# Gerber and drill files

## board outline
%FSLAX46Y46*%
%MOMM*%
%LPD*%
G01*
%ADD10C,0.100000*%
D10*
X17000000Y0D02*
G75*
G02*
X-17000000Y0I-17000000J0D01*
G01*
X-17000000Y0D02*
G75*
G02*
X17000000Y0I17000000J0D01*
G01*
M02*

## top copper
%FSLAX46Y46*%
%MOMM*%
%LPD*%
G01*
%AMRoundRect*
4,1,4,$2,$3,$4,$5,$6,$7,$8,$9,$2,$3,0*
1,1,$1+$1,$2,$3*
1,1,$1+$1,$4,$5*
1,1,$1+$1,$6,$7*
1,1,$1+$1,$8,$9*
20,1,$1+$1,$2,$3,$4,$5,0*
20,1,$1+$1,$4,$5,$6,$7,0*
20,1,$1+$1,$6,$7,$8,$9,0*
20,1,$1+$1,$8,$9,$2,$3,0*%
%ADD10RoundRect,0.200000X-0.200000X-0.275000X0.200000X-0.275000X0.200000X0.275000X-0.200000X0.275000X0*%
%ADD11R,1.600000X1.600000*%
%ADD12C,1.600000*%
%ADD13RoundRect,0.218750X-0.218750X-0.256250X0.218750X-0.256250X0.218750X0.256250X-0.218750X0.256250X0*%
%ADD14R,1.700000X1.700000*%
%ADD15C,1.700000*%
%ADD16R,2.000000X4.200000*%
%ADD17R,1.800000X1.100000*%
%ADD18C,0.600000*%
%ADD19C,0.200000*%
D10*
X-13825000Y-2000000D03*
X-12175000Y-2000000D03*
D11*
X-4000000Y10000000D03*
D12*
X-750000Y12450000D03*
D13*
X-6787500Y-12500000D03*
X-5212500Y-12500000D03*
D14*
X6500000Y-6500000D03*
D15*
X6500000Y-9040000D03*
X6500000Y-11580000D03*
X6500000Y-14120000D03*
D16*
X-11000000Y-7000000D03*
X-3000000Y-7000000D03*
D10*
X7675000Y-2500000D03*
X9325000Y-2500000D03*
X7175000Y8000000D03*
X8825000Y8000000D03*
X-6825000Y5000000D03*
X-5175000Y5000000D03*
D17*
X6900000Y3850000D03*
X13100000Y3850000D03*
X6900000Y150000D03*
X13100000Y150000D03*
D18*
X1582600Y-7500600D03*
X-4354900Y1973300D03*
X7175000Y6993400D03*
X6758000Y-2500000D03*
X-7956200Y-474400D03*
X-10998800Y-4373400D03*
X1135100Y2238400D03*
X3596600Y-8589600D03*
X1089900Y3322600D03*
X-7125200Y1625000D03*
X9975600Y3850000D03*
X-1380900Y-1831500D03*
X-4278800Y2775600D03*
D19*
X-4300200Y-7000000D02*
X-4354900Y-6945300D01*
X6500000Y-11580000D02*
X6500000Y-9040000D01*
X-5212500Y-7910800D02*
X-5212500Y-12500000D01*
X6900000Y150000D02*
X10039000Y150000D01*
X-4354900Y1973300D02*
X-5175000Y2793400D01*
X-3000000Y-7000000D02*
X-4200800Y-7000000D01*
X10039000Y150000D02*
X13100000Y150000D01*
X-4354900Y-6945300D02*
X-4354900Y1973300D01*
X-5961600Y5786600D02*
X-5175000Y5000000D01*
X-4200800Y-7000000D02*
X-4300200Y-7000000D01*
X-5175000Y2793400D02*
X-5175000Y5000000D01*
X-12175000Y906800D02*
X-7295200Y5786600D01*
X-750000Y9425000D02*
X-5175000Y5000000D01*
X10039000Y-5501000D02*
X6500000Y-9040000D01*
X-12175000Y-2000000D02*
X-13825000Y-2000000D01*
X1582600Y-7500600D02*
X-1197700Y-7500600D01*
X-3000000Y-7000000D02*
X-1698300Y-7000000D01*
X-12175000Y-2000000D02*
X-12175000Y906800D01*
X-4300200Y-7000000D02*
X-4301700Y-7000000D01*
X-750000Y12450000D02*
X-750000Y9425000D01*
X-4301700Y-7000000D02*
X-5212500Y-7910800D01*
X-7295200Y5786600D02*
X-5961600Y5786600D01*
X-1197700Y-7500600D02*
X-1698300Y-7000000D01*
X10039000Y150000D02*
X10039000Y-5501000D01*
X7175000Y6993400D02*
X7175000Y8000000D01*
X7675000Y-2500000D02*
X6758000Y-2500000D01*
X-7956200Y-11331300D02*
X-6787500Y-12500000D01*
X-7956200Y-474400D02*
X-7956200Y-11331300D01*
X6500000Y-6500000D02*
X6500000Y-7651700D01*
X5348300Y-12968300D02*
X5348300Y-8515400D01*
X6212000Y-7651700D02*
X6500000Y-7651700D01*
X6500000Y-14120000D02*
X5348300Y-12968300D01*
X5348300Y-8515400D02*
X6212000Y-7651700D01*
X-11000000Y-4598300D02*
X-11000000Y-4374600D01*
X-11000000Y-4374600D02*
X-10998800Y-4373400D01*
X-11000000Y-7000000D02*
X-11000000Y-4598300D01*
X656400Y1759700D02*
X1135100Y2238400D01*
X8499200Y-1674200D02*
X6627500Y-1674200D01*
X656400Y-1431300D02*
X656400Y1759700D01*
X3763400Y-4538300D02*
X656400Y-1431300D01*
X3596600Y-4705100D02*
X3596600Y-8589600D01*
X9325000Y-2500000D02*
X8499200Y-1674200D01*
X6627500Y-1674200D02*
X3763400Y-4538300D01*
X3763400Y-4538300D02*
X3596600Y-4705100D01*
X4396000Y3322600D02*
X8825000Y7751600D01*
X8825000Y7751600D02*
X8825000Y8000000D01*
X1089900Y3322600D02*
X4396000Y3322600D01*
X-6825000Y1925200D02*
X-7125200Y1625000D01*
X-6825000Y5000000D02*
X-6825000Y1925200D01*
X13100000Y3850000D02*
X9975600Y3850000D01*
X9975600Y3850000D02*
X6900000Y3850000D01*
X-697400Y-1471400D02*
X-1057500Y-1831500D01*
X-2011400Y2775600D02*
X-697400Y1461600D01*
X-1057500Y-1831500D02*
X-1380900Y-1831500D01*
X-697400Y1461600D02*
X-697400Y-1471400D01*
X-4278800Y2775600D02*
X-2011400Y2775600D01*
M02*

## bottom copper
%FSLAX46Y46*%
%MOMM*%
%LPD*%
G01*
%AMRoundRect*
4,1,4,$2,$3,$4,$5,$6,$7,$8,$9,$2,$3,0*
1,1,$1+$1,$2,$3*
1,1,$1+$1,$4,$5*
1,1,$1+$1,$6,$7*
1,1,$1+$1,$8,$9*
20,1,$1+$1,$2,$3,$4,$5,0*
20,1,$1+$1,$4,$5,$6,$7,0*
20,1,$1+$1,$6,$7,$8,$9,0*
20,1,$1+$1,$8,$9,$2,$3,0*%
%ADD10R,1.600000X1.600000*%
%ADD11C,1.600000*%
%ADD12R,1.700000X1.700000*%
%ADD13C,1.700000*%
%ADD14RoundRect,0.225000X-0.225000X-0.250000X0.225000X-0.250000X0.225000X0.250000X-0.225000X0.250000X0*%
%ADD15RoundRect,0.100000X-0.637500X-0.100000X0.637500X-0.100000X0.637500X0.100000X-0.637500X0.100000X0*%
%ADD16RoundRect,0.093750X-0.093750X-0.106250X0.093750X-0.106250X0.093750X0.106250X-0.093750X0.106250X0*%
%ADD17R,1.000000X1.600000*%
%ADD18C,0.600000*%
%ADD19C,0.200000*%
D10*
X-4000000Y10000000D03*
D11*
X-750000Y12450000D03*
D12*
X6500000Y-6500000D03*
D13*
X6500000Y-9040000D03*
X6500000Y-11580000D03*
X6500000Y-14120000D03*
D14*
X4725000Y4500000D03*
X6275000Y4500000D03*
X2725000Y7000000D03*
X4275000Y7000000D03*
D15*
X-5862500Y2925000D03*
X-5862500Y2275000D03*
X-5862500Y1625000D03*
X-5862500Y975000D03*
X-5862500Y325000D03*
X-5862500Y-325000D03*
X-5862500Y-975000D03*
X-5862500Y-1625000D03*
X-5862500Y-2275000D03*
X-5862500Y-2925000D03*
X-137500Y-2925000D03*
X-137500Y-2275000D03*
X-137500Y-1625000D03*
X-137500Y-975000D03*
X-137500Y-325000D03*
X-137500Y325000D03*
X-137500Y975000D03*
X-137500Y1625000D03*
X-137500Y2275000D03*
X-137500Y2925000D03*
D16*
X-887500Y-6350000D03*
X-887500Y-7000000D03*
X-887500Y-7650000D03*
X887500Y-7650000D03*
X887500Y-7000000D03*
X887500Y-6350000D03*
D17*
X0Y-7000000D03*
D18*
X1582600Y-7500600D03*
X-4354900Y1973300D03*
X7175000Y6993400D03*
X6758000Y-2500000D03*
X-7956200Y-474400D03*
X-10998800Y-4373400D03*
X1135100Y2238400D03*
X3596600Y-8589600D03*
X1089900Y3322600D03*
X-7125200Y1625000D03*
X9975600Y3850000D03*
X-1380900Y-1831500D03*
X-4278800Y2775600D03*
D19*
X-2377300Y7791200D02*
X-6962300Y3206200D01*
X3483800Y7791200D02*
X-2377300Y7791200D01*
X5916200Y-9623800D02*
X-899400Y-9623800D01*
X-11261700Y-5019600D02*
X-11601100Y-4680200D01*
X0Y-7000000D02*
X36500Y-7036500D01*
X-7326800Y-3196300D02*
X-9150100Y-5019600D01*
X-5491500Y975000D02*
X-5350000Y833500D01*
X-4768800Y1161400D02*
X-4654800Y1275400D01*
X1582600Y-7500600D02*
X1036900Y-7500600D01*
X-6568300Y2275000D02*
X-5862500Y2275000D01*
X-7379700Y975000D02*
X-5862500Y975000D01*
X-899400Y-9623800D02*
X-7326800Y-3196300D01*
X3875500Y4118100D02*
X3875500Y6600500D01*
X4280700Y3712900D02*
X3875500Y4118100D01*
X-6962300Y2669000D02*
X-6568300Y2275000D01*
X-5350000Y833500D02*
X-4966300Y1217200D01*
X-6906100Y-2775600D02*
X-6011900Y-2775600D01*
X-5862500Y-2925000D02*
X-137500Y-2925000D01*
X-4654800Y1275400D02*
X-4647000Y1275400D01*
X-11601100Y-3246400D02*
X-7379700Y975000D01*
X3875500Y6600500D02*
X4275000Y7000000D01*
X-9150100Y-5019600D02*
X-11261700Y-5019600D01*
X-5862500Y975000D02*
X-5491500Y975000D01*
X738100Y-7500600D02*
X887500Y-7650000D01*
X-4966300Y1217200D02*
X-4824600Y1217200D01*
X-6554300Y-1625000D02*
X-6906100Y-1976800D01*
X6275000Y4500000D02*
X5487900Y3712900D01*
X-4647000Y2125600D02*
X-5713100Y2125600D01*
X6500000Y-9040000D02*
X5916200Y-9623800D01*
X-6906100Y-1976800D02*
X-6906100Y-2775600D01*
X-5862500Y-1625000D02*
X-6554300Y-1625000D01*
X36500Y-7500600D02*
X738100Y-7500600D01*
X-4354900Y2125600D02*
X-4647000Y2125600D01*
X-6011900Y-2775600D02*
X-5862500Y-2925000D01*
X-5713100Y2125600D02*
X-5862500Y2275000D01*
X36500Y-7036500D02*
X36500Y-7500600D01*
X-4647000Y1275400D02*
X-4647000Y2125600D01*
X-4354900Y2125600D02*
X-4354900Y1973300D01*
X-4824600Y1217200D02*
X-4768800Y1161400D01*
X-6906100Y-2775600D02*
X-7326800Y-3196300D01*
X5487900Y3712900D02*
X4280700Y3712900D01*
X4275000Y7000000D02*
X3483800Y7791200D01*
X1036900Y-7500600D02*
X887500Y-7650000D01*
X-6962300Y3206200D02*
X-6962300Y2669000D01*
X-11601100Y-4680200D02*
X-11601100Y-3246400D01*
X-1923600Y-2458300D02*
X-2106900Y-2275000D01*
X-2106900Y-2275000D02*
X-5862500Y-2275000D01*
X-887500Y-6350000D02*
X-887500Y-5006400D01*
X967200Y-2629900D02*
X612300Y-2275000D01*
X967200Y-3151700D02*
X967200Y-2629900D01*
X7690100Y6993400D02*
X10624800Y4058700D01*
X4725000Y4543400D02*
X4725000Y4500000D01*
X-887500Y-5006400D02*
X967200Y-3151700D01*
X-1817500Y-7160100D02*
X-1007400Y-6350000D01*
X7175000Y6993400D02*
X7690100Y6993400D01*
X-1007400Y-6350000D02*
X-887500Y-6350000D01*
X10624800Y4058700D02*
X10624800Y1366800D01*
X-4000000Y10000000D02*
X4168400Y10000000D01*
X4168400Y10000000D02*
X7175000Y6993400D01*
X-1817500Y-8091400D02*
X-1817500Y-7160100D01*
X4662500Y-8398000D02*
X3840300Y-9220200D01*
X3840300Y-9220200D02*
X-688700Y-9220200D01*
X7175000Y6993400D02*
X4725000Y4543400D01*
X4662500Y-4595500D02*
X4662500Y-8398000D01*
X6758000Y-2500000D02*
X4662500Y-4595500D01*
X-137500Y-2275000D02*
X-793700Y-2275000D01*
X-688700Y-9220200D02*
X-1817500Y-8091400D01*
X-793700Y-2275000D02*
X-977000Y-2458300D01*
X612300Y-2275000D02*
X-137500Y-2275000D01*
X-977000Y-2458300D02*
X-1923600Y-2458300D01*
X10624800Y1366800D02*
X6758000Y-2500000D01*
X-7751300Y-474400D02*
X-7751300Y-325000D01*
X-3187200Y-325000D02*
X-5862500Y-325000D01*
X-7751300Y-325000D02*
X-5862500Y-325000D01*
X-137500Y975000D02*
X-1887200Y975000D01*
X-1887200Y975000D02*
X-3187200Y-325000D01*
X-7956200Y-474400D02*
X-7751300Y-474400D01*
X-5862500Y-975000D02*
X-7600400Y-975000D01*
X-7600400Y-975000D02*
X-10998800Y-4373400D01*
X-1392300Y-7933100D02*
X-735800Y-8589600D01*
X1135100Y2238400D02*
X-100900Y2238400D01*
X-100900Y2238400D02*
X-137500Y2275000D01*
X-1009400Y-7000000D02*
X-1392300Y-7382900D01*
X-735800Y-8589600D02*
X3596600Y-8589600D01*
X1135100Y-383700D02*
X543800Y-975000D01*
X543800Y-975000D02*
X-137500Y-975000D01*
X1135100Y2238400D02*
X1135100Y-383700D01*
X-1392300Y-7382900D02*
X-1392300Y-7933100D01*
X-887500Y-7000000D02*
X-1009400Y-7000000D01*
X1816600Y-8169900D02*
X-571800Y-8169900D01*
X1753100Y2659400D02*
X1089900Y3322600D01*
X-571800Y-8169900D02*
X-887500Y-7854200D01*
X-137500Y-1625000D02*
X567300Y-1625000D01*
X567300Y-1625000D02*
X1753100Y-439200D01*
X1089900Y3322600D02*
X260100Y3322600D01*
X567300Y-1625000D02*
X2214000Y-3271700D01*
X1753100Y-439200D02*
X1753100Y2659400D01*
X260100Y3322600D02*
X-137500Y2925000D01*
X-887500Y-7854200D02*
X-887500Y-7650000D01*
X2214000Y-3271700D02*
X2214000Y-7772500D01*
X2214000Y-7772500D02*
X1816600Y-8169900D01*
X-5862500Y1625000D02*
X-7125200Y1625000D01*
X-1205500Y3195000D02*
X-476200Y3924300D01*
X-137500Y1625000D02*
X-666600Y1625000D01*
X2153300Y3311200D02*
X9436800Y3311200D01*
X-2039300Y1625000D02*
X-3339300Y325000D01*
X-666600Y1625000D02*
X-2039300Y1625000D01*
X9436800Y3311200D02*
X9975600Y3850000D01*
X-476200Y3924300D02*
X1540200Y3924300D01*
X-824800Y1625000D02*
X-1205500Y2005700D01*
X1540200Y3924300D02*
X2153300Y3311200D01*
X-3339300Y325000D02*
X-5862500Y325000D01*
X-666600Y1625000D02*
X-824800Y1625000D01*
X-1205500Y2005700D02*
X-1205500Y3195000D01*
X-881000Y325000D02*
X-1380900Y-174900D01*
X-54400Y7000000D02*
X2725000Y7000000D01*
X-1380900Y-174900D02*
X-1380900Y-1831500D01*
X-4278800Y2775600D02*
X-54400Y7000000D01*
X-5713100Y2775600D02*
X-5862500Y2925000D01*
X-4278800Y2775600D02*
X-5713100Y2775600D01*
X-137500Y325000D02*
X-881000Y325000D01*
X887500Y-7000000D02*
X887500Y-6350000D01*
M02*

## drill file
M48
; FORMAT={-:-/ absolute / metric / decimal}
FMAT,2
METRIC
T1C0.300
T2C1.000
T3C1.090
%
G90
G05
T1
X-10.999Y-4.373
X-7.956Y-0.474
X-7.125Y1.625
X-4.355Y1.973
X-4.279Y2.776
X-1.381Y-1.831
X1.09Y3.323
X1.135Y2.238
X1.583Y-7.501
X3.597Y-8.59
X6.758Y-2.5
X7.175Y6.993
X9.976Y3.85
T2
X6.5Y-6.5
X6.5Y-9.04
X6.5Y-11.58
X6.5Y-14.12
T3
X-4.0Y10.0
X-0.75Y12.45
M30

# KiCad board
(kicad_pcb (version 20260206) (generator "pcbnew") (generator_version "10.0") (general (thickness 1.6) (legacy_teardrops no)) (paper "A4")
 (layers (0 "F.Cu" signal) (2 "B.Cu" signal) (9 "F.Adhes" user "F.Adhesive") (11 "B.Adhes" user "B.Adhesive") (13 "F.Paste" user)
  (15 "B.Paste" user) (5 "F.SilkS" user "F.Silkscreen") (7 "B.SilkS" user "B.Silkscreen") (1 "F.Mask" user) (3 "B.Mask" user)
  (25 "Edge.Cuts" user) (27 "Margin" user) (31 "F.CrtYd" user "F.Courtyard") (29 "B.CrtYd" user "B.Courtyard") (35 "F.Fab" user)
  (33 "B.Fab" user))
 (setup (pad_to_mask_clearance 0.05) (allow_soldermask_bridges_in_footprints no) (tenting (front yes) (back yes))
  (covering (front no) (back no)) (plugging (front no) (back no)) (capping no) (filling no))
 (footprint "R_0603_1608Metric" (layer "F.Cu") (at -13 2 90)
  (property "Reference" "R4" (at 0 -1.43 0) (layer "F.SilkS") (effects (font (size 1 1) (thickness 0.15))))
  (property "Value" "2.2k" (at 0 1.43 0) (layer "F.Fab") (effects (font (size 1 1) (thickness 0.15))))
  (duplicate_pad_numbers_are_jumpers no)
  (pad "1" smd roundrect (at 0 -0.825) (size 0.8 0.95) (layers "F.Cu" "F.Mask" "F.Paste") (roundrect_rratio 0.25) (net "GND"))
  (pad "2" smd roundrect (at 0 0.825) (size 0.8 0.95) (layers "F.Cu" "F.Mask" "F.Paste") (roundrect_rratio 0.25) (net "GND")))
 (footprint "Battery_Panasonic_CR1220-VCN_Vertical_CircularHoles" (layer "F.Cu") (at -4 -10)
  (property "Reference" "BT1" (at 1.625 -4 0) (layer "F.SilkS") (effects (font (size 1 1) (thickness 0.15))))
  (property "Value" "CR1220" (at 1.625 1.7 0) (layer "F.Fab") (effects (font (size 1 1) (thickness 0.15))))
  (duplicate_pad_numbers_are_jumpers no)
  (pad "1" thru_hole rect (at 0 0 90) (size 1.6 1.6) (drill 1.09) (layers "*.Cu" "*.Mask") (remove_unused_layers no) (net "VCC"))
  (pad "2" thru_hole circle (at 3.25 -2.45) (size 1.6 1.6) (drill 1.09) (layers "*.Cu" "*.Mask") (remove_unused_layers no) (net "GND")))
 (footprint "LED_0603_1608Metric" (layer "F.Cu") (at -6 12.5)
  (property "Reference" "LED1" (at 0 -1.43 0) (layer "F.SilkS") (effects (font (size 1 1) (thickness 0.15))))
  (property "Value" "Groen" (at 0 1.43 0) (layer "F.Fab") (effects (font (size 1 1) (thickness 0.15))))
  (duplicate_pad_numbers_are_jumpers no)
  (pad "1" smd roundrect (at -0.7875 0) (size 0.875 0.95) (layers "F.Cu" "F.Mask" "F.Paste") (roundrect_rratio 0.25) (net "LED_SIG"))
  (pad "2" smd roundrect (at 0.7875 0) (size 0.875 0.95) (layers "F.Cu" "F.Mask" "F.Paste") (roundrect_rratio 0.25) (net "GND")))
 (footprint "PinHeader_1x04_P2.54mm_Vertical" (layer "F.Cu") (at 6.5 6.5)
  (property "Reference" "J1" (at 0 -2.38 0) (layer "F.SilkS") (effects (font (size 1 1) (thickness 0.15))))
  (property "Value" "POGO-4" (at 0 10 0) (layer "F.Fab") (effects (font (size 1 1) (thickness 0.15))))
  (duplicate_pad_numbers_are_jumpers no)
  (pad "1" thru_hole rect (at 0 0) (size 1.7 1.7) (drill 1) (layers "*.Cu" "*.Mask") (remove_unused_layers no) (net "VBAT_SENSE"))
  (pad "2" thru_hole circle (at 0 2.54) (size 1.7 1.7) (drill 1) (layers "*.Cu" "*.Mask") (remove_unused_layers no) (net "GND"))
  (pad "3" thru_hole circle (at 0 5.08) (size 1.7 1.7) (drill 1) (layers "*.Cu" "*.Mask") (remove_unused_layers no) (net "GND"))
  (pad "4" thru_hole circle (at 0 7.62) (size 1.7 1.7) (drill 1) (layers "*.Cu" "*.Mask") (remove_unused_layers no) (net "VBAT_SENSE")))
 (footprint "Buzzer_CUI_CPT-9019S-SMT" (layer "F.Cu") (at -7 7)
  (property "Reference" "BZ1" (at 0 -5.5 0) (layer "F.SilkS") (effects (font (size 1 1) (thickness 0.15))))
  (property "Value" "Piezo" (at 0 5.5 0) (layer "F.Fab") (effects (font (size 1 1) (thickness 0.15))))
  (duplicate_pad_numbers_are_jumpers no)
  (pad "1" smd rect (at -4 0) (size 2 4.2) (layers "F.Cu" "F.Mask" "F.Paste") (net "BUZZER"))
  (pad "2" smd rect (at 4 0) (size 2 4.2) (layers "F.Cu" "F.Mask" "F.Paste") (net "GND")))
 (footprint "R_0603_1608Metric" (layer "F.Cu") (at 8.5 2.5 90)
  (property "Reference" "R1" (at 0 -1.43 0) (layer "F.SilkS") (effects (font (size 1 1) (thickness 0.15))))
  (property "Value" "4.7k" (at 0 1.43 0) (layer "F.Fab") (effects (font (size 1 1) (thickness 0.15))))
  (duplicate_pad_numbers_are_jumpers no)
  (pad "1" smd roundrect (at 0 -0.825) (size 0.8 0.95) (layers "F.Cu" "F.Mask" "F.Paste") (roundrect_rratio 0.25) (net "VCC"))
  (pad "2" smd roundrect (at 0 0.825) (size 0.8 0.95) (layers "F.Cu" "F.Mask" "F.Paste") (roundrect_rratio 0.25) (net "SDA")))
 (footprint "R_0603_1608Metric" (layer "F.Cu") (at 8 -8 90)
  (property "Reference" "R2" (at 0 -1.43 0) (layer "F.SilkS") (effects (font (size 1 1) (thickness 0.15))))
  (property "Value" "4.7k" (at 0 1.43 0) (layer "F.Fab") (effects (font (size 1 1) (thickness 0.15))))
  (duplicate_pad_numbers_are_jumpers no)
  (pad "1" smd roundrect (at 0 -0.825) (size 0.8 0.95) (layers "F.Cu" "F.Mask" "F.Paste") (roundrect_rratio 0.25) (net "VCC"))
  (pad "2" smd roundrect (at 0 0.825) (size 0.8 0.95) (layers "F.Cu" "F.Mask" "F.Paste") (roundrect_rratio 0.25) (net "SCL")))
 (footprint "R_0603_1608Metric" (layer "F.Cu") (at -6 -5)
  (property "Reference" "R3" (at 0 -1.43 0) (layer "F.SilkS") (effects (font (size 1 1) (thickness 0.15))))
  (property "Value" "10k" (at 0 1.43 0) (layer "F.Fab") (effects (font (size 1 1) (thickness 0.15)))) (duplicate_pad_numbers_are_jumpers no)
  (pad "1" smd roundrect (at -0.825 0) (size 0.8 0.95) (layers "F.Cu" "F.Mask" "F.Paste") (roundrect_rratio 0.25) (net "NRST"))
  (pad "2" smd roundrect (at 0.825 0) (size 0.8 0.95) (layers "F.Cu" "F.Mask" "F.Paste") (roundrect_rratio 0.25) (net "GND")))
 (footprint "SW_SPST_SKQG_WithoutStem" (layer "F.Cu") (at 10 -2)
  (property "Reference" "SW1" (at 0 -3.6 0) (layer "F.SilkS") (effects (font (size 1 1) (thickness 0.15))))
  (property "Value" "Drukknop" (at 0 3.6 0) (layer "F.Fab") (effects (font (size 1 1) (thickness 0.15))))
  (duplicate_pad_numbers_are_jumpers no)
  (pad "1" smd rect (at -3.1 -1.85) (size 1.8 1.1) (layers "F.Cu" "F.Mask" "F.Paste") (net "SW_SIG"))
  (pad "1" smd rect (at 3.1 -1.85) (size 1.8 1.1) (layers "F.Cu" "F.Mask" "F.Paste") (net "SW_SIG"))
  (pad "2" smd rect (at -3.1 1.85) (size 1.8 1.1) (layers "F.Cu" "F.Mask" "F.Paste") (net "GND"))
  (pad "2" smd rect (at 3.1 1.85) (size 1.8 1.1) (layers "F.Cu" "F.Mask" "F.Paste") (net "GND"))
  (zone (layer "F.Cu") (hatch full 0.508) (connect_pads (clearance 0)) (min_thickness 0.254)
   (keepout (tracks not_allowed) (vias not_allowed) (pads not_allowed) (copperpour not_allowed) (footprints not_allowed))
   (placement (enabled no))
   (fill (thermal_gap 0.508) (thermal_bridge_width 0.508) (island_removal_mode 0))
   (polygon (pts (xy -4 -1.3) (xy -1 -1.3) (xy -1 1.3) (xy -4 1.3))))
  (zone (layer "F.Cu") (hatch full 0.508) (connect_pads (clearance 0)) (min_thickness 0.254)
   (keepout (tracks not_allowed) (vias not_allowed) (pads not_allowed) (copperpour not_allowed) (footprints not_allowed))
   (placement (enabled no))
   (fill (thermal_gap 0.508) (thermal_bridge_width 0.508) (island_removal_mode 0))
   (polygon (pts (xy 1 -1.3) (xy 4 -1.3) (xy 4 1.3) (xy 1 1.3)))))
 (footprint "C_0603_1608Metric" (layer "B.Cu") (at 5.5 -4.5 90)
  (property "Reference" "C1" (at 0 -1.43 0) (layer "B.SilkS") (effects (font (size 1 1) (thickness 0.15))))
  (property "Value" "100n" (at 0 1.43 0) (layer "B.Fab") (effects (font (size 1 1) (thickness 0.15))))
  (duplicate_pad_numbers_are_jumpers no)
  (pad "1" smd roundrect (at 0 -0.775) (size 0.9 0.95) (layers "B.Cu" "B.Mask" "B.Paste") (roundrect_rratio 0.25) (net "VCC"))
  (pad "2" smd roundrect (at 0 0.775) (size 0.9 0.95) (layers "B.Cu" "B.Mask" "B.Paste") (roundrect_rratio 0.25) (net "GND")))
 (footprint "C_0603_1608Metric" (layer "B.Cu") (at 3.5 -7 90)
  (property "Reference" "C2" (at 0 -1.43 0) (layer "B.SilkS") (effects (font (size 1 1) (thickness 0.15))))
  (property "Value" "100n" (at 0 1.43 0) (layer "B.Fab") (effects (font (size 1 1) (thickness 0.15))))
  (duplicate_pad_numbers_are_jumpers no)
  (pad "1" smd roundrect (at 0 -0.775) (size 0.9 0.95) (layers "B.Cu" "B.Mask" "B.Paste") (roundrect_rratio 0.25) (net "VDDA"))
  (pad "2" smd roundrect (at 0 0.775) (size 0.9 0.95) (layers "B.Cu" "B.Mask" "B.Paste") (roundrect_rratio 0.25) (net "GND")))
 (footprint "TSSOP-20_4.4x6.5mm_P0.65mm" (layer "B.Cu") (at -3 0 180)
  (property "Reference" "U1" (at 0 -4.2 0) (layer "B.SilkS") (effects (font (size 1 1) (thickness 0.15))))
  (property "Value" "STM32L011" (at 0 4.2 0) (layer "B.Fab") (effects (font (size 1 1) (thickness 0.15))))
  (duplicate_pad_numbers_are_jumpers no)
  (pad "1" smd roundrect (at 2.8625 2.925) (size 1.475 0.4) (layers "B.Cu" "B.Mask" "B.Paste") (roundrect_rratio 0.25) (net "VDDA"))
  (pad "2" smd roundrect (at 2.8625 2.275) (size 1.475 0.4) (layers "B.Cu" "B.Mask" "B.Paste") (roundrect_rratio 0.25) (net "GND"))
  (pad "3" smd roundrect (at 2.8625 1.625) (size 1.475 0.4) (layers "B.Cu" "B.Mask" "B.Paste") (roundrect_rratio 0.25) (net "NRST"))
  (pad "4" smd roundrect (at 2.8625 0.975) (size 1.475 0.4) (layers "B.Cu" "B.Mask" "B.Paste") (roundrect_rratio 0.25) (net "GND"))
  (pad "5" smd roundrect (at 2.8625 0.325) (size 1.475 0.4) (layers "B.Cu" "B.Mask" "B.Paste") (roundrect_rratio 0.25) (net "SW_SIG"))
  (pad "6" smd roundrect (at 2.8625 -0.325) (size 1.475 0.4) (layers "B.Cu" "B.Mask" "B.Paste") (roundrect_rratio 0.25) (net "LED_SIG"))
  (pad "7" smd roundrect (at 2.8625 -0.975) (size 1.475 0.4) (layers "B.Cu" "B.Mask" "B.Paste") (roundrect_rratio 0.25) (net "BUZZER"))
  (pad "8" smd roundrect (at 2.8625 -1.625) (size 1.475 0.4) (layers "B.Cu" "B.Mask" "B.Paste") (roundrect_rratio 0.25) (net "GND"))
  (pad "9" smd roundrect (at 2.8625 -2.275) (size 1.475 0.4) (layers "B.Cu" "B.Mask" "B.Paste") (roundrect_rratio 0.25) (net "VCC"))
  (pad "10" smd roundrect (at 2.8625 -2.925) (size 1.475 0.4) (layers "B.Cu" "B.Mask" "B.Paste") (roundrect_rratio 0.25) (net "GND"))
  (pad "11" smd roundrect (at -2.8625 -2.925) (size 1.475 0.4) (layers "B.Cu" "B.Mask" "B.Paste") (roundrect_rratio 0.25) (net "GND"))
  (pad "12" smd roundrect (at -2.8625 -2.275) (size 1.475 0.4) (layers "B.Cu" "B.Mask" "B.Paste") (roundrect_rratio 0.25) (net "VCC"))
  (pad "13" smd roundrect (at -2.8625 -1.625) (size 1.475 0.4) (layers "B.Cu" "B.Mask" "B.Paste") (roundrect_rratio 0.25) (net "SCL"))
  (pad "14" smd roundrect (at -2.8625 -0.975) (size 1.475 0.4) (layers "B.Cu" "B.Mask" "B.Paste") (roundrect_rratio 0.25) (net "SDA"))
  (pad "15" smd roundrect (at -2.8625 -0.325) (size 1.475 0.4) (layers "B.Cu" "B.Mask" "B.Paste") (roundrect_rratio 0.25) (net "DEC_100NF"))
  (pad "16" smd roundrect (at -2.8625 0.325) (size 1.475 0.4) (layers "B.Cu" "B.Mask" "B.Paste") (roundrect_rratio 0.25) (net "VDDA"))
  (pad "17" smd roundrect (at -2.8625 0.975) (size 1.475 0.4) (layers "B.Cu" "B.Mask" "B.Paste") (roundrect_rratio 0.25) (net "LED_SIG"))
  (pad "18" smd roundrect (at -2.8625 1.625) (size 1.475 0.4) (layers "B.Cu" "B.Mask" "B.Paste") (roundrect_rratio 0.25) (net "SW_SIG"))
  (pad "19" smd roundrect (at -2.8625 2.275) (size 1.475 0.4) (layers "B.Cu" "B.Mask" "B.Paste") (roundrect_rratio 0.25) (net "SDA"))
  (pad "20" smd roundrect (at -2.8625 2.925) (size 1.475 0.4) (layers "B.Cu" "B.Mask" "B.Paste") (roundrect_rratio 0.25) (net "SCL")))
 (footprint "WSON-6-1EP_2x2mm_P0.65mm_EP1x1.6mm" (layer "B.Cu") (at 0 7)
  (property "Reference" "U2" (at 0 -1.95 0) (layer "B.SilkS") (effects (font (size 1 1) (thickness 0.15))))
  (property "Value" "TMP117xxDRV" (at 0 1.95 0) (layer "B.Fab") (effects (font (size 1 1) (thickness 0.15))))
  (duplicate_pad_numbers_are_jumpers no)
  (pad "" smd roundrect (at 0 -0.4) (size 0.81 0.64) (layers "B.Paste") (roundrect_rratio 0.25))
  (pad "" smd roundrect (at 0 0.4) (size 0.81 0.64) (layers "B.Paste") (roundrect_rratio 0.25))
  (pad "1" smd roundrect (at -0.8875 -0.65) (size 0.375 0.4) (layers "B.Cu" "B.Mask" "B.Paste") (roundrect_rratio 0.25) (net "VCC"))
  (pad "2" smd roundrect (at -0.8875 0) (size 0.375 0.4) (layers "B.Cu" "B.Mask" "B.Paste") (roundrect_rratio 0.25) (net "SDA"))
  (pad "3" smd roundrect (at -0.8875 0.65) (size 0.375 0.4) (layers "B.Cu" "B.Mask" "B.Paste") (roundrect_rratio 0.25) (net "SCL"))
  (pad "4" smd roundrect (at 0.8875 0.65) (size 0.375 0.4) (layers "B.Cu" "B.Mask" "B.Paste") (roundrect_rratio 0.25) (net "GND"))
  (pad "5" smd roundrect (at 0.8875 0) (size 0.375 0.4) (layers "B.Cu" "B.Mask" "B.Paste") (roundrect_rratio 0.25) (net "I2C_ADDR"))
  (pad "6" smd roundrect (at 0.8875 -0.65) (size 0.375 0.4) (layers "B.Cu" "B.Mask" "B.Paste") (roundrect_rratio 0.25) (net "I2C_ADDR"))
  (pad "7" smd rect (at 0 0) (size 1 1.6) (layers "B.Cu" "B.Mask") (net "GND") (zone_connect 2)))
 (gr_circle (center 0 0) (end 17 0) (stroke (width 0.1) (type solid)) (fill no) (layer "Edge.Cuts"))
 (segment (start -4.3002 7) (end -4.3549 6.9453) (width 0.2) (layer "F.Cu") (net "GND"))
 (segment (start 6.5 11.58) (end 6.5 9.04) (width 0.2) (layer "F.Cu") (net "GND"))
 (segment (start -5.2125 7.9108) (end -5.2125 12.5) (width 0.2) (layer "F.Cu") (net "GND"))
 (segment (start 6.9 -0.15) (end 10.039 -0.15) (width 0.2) (layer "F.Cu") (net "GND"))
 (segment (start -4.3549 -1.9733) (end -5.175 -2.7934) (width 0.2) (layer "F.Cu") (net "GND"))
 (segment (start -3 7) (end -4.2008 7) (width 0.2) (layer "F.Cu") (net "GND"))
 (segment (start 10.039 -0.15) (end 13.1 -0.15) (width 0.2) (layer "F.Cu") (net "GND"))
 (segment (start -4.3549 6.9453) (end -4.3549 -1.9733) (width 0.2) (layer "F.Cu") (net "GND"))
 (segment (start -5.9616 -5.7866) (end -5.175 -5) (width 0.2) (layer "F.Cu") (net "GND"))
 (segment (start -4.2008 7) (end -4.3002 7) (width 0.2) (layer "F.Cu") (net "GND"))
 (segment (start -5.175 -2.7934) (end -5.175 -5) (width 0.2) (layer "F.Cu") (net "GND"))
 (segment (start -12.175 -0.9068) (end -7.2952 -5.7866) (width 0.2) (layer "F.Cu") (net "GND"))
 (segment (start -0.75 -9.425) (end -5.175 -5) (width 0.2) (layer "F.Cu") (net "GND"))
 (segment (start 10.039 5.501) (end 6.5 9.04) (width 0.2) (layer "F.Cu") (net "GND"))
 (segment (start -12.175 2) (end -13.825 2) (width 0.2) (layer "F.Cu") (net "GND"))
 (segment (start 1.5826 7.5006) (end -1.1977 7.5006) (width 0.2) (layer "F.Cu") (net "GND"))
 (segment (start -3 7) (end -1.6983 7) (width 0.2) (layer "F.Cu") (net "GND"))
 (segment (start -12.175 2) (end -12.175 -0.9068) (width 0.2) (layer "F.Cu") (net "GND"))
 (segment (start -4.3002 7) (end -4.3017 7) (width 0.2) (layer "F.Cu") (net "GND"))
 (segment (start -0.75 -12.45) (end -0.75 -9.425) (width 0.2) (layer "F.Cu") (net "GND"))
 (segment (start -4.3017 7) (end -5.2125 7.9108) (width 0.2) (layer "F.Cu") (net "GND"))
 (segment (start -7.2952 -5.7866) (end -5.9616 -5.7866) (width 0.2) (layer "F.Cu") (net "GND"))
 (segment (start -1.1977 7.5006) (end -1.6983 7) (width 0.2) (layer "F.Cu") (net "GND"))
 (segment (start 10.039 -0.15) (end 10.039 5.501) (width 0.2) (layer "F.Cu") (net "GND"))
 (via (at 1.5826 7.5006) (size 0.6) (drill 0.3) (layers "F.Cu" "B.Cu") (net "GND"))
 (via (at -4.3549 -1.9733) (size 0.6) (drill 0.3) (layers "F.Cu" "B.Cu") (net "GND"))
 (segment (start -2.3773 -7.7912) (end -6.9623 -3.2062) (width 0.2) (layer "B.Cu") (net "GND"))
 (segment (start 3.4838 -7.7912) (end -2.3773 -7.7912) (width 0.2) (layer "B.Cu") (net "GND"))
 (segment (start 5.9162 9.6238) (end -0.8994 9.6238) (width 0.2) (layer "B.Cu") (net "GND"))
 (segment (start -11.2617 5.0196) (end -11.6011 4.6802) (width 0.2) (layer "B.Cu") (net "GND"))
 (segment (start 0 7) (end 0.0365 7.0365) (width 0.2) (layer "B.Cu") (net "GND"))
 (segment (start -7.3268 3.1963) (end -9.1501 5.0196) (width 0.2) (layer "B.Cu") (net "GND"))
 (segment (start -5.4915 -0.975) (end -5.35 -0.8335) (width 0.2) (layer "B.Cu") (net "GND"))
 (segment (start -4.7688 -1.1614) (end -4.6548 -1.2754) (width 0.2) (layer "B.Cu") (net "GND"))
 (segment (start 1.5826 7.5006) (end 1.0369 7.5006) (width 0.2) (layer "B.Cu") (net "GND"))
 (segment (start -6.5683 -2.275) (end -5.8625 -2.275) (width 0.2) (layer "B.Cu") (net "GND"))
 (segment (start -7.3797 -0.975) (end -5.8625 -0.975) (width 0.2) (layer "B.Cu") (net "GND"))
 (segment (start -0.8994 9.6238) (end -7.3268 3.1963) (width 0.2) (layer "B.Cu") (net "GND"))
 (segment (start 3.8755 -4.1181) (end 3.8755 -6.6005) (width 0.2) (layer "B.Cu") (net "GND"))
 (segment (start 4.2807 -3.7129) (end 3.8755 -4.1181) (width 0.2) (layer "B.Cu") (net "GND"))
 (segment (start -6.9623 -2.669) (end -6.5683 -2.275) (width 0.2) (layer "B.Cu") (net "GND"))
 (segment (start -5.35 -0.8335) (end -4.9663 -1.2172) (width 0.2) (layer "B.Cu") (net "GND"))
 (segment (start -6.9061 2.7756) (end -6.0119 2.7756) (width 0.2) (layer "B.Cu") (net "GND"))
 (segment (start -5.8625 2.925) (end -0.1375 2.925) (width 0.2) (layer "B.Cu") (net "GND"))
 (segment (start -4.6548 -1.2754) (end -4.647 -1.2754) (width 0.2) (layer "B.Cu") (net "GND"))
 (segment (start -11.6011 3.2464) (end -7.3797 -0.975) (width 0.2) (layer "B.Cu") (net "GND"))
 (segment (start 3.8755 -6.6005) (end 4.275 -7) (width 0.2) (layer "B.Cu") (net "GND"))
 (segment (start -9.1501 5.0196) (end -11.2617 5.0196) (width 0.2) (layer "B.Cu") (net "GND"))
 (segment (start -5.8625 -0.975) (end -5.4915 -0.975) (width 0.2) (layer "B.Cu") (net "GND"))
 (segment (start 0.7381 7.5006) (end 0.8875 7.65) (width 0.2) (layer "B.Cu") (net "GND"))
 (segment (start -4.9663 -1.2172) (end -4.8246 -1.2172) (width 0.2) (layer "B.Cu") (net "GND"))
 (segment (start -6.5543 1.625) (end -6.9061 1.9768) (width 0.2) (layer "B.Cu") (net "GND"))
 (segment (start 6.275 -4.5) (end 5.4879 -3.7129) (width 0.2) (layer "B.Cu") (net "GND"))
 (segment (start -4.647 -2.1256) (end -5.7131 -2.1256) (width 0.2) (layer "B.Cu") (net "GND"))
 (segment (start 6.5 9.04) (end 5.9162 9.6238) (width 0.2) (layer "B.Cu") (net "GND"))
 (segment (start -6.9061 1.9768) (end -6.9061 2.7756) (width 0.2) (layer "B.Cu") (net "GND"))
 (segment (start -5.8625 1.625) (end -6.5543 1.625) (width 0.2) (layer "B.Cu") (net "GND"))
 (segment (start 0.0365 7.5006) (end 0.7381 7.5006) (width 0.2) (layer "B.Cu") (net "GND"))
 (segment (start -4.3549 -2.1256) (end -4.647 -2.1256) (width 0.2) (layer "B.Cu") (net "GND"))
 (segment (start -6.0119 2.7756) (end -5.8625 2.925) (width 0.2) (layer "B.Cu") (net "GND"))
 (segment (start -5.7131 -2.1256) (end -5.8625 -2.275) (width 0.2) (layer "B.Cu") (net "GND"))
 (segment (start 0.0365 7.0365) (end 0.0365 7.5006) (width 0.2) (layer "B.Cu") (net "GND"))
 (segment (start -4.647 -1.2754) (end -4.647 -2.1256) (width 0.2) (layer "B.Cu") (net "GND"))
 (segment (start -4.3549 -2.1256) (end -4.3549 -1.9733) (width 0.2) (layer "B.Cu") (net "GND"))
 (segment (start -4.8246 -1.2172) (end -4.7688 -1.1614) (width 0.2) (layer "B.Cu") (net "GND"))
 (segment (start -6.9061 2.7756) (end -7.3268 3.1963) (width 0.2) (layer "B.Cu") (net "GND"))
 (segment (start 5.4879 -3.7129) (end 4.2807 -3.7129) (width 0.2) (layer "B.Cu") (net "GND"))
 (segment (start 4.275 -7) (end 3.4838 -7.7912) (width 0.2) (layer "B.Cu") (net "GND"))
 (segment (start 1.0369 7.5006) (end 0.8875 7.65) (width 0.2) (layer "B.Cu") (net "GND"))
 (segment (start -6.9623 -3.2062) (end -6.9623 -2.669) (width 0.2) (layer "B.Cu") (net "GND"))
 (segment (start -11.6011 4.6802) (end -11.6011 3.2464) (width 0.2) (layer "B.Cu") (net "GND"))
 (segment (start 7.175 -6.9934) (end 7.175 -8) (width 0.2) (layer "F.Cu") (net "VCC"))
 (segment (start 7.675 2.5) (end 6.758 2.5) (width 0.2) (layer "F.Cu") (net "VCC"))
 (via (at 7.175 -6.9934) (size 0.6) (drill 0.3) (layers "F.Cu" "B.Cu") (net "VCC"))
 (via (at 6.758 2.5) (size 0.6) (drill 0.3) (layers "F.Cu" "B.Cu") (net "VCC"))
 (segment (start -1.9236 2.4583) (end -2.1069 2.275) (width 0.2) (layer "B.Cu") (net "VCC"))
 (segment (start -2.1069 2.275) (end -5.8625 2.275) (width 0.2) (layer "B.Cu") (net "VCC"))
 (segment (start -0.8875 6.35) (end -0.8875 5.0064) (width 0.2) (layer "B.Cu") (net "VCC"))
 (segment (start 0.9672 2.6299) (end 0.6123 2.275) (width 0.2) (layer "B.Cu") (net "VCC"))
 (segment (start 0.9672 3.1517) (end 0.9672 2.6299) (width 0.2) (layer "B.Cu") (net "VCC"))
 (segment (start 7.6901 -6.9934) (end 10.6248 -4.0587) (width 0.2) (layer "B.Cu") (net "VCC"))
 (segment (start 4.725 -4.5434) (end 4.725 -4.5) (width 0.2) (layer "B.Cu") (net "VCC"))
 (segment (start -0.8875 5.0064) (end 0.9672 3.1517) (width 0.2) (layer "B.Cu") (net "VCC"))
 (segment (start -1.8175 7.1601) (end -1.0074 6.35) (width 0.2) (layer "B.Cu") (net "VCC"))
 (segment (start 7.175 -6.9934) (end 7.6901 -6.9934) (width 0.2) (layer "B.Cu") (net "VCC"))
 (segment (start -1.0074 6.35) (end -0.8875 6.35) (width 0.2) (layer "B.Cu") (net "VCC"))
 (segment (start 10.6248 -4.0587) (end 10.6248 -1.3668) (width 0.2) (layer "B.Cu") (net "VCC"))
 (segment (start -4 -10) (end 4.1684 -10) (width 0.2) (layer "B.Cu") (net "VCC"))
 (segment (start 4.1684 -10) (end 7.175 -6.9934) (width 0.2) (layer "B.Cu") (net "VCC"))
 (segment (start -1.8175 8.0914) (end -1.8175 7.1601) (width 0.2) (layer "B.Cu") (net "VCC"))
 (segment (start 4.6625 8.398) (end 3.8403 9.2202) (width 0.2) (layer "B.Cu") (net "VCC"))
 (segment (start 3.8403 9.2202) (end -0.6887 9.2202) (width 0.2) (layer "B.Cu") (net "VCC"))
 (segment (start 7.175 -6.9934) (end 4.725 -4.5434) (width 0.2) (layer "B.Cu") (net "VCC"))
 (segment (start 4.6625 4.5955) (end 4.6625 8.398) (width 0.2) (layer "B.Cu") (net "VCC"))
 (segment (start 6.758 2.5) (end 4.6625 4.5955) (width 0.2) (layer "B.Cu") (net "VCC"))
 (segment (start -0.1375 2.275) (end -0.7937 2.275) (width 0.2) (layer "B.Cu") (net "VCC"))
 (segment (start -0.6887 9.2202) (end -1.8175 8.0914) (width 0.2) (layer "B.Cu") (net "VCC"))
 (segment (start -0.7937 2.275) (end -0.977 2.4583) (width 0.2) (layer "B.Cu") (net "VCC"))
 (segment (start 0.6123 2.275) (end -0.1375 2.275) (width 0.2) (layer "B.Cu") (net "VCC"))
 (segment (start -0.977 2.4583) (end -1.9236 2.4583) (width 0.2) (layer "B.Cu") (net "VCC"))
 (segment (start 10.6248 -1.3668) (end 6.758 2.5) (width 0.2) (layer "B.Cu") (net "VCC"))
 (segment (start -7.9562 11.3313) (end -6.7875 12.5) (width 0.2) (layer "F.Cu") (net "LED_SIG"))
 (segment (start -7.9562 0.4744) (end -7.9562 11.3313) (width 0.2) (layer "F.Cu") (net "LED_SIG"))
 (via (at -7.9562 0.4744) (size 0.6) (drill 0.3) (layers "F.Cu" "B.Cu") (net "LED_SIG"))
 (segment (start -7.7513 0.4744) (end -7.7513 0.325) (width 0.2) (layer "B.Cu") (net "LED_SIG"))
 (segment (start -3.1872 0.325) (end -5.8625 0.325) (width 0.2) (layer "B.Cu") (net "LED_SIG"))
 (segment (start -7.7513 0.325) (end -5.8625 0.325) (width 0.2) (layer "B.Cu") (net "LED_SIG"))
 (segment (start -0.1375 -0.975) (end -1.8872 -0.975) (width 0.2) (layer "B.Cu") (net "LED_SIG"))
 (segment (start -1.8872 -0.975) (end -3.1872 0.325) (width 0.2) (layer "B.Cu") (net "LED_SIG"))
 (segment (start -7.9562 0.4744) (end -7.7513 0.4744) (width 0.2) (layer "B.Cu") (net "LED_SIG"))
 (segment (start 6.5 6.5) (end 6.5 7.6517) (width 0.2) (layer "F.Cu") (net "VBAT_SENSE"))
 (segment (start 5.3483 12.9683) (end 5.3483 8.5154) (width 0.2) (layer "F.Cu") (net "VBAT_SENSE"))
 (segment (start 6.212 7.6517) (end 6.5 7.6517) (width 0.2) (layer "F.Cu") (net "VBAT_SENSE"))
 (segment (start 6.5 14.12) (end 5.3483 12.9683) (width 0.2) (layer "F.Cu") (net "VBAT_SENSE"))
 (segment (start 5.3483 8.5154) (end 6.212 7.6517) (width 0.2) (layer "F.Cu") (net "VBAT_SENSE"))
 (segment (start -11 4.5983) (end -11 4.3746) (width 0.2) (layer "F.Cu") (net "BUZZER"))
 (segment (start -11 4.3746) (end -10.9988 4.3734) (width 0.2) (layer "F.Cu") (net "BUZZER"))
 (segment (start -11 7) (end -11 4.5983) (width 0.2) (layer "F.Cu") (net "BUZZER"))
 (via (at -10.9988 4.3734) (size 0.6) (drill 0.3) (layers "F.Cu" "B.Cu") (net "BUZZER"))
 (segment (start -5.8625 0.975) (end -7.6004 0.975) (width 0.2) (layer "B.Cu") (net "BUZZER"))
 (segment (start -7.6004 0.975) (end -10.9988 4.3734) (width 0.2) (layer "B.Cu") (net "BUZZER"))
 (segment (start 0.6564 -1.7597) (end 1.1351 -2.2384) (width 0.2) (layer "F.Cu") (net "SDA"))
 (segment (start 8.4992 1.6742) (end 6.6275 1.6742) (width 0.2) (layer "F.Cu") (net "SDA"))
 (segment (start 0.6564 1.4313) (end 0.6564 -1.7597) (width 0.2) (layer "F.Cu") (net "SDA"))
 (segment (start 3.7634 4.5383) (end 0.6564 1.4313) (width 0.2) (layer "F.Cu") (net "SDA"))
 (segment (start 3.5966 4.7051) (end 3.5966 8.5896) (width 0.2) (layer "F.Cu") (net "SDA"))
 (segment (start 9.325 2.5) (end 8.4992 1.6742) (width 0.2) (layer "F.Cu") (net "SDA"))
 (segment (start 6.6275 1.6742) (end 3.7634 4.5383) (width 0.2) (layer "F.Cu") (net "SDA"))
 (segment (start 3.7634 4.5383) (end 3.5966 4.7051) (width 0.2) (layer "F.Cu") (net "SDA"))
 (via (at 1.1351 -2.2384) (size 0.6) (drill 0.3) (layers "F.Cu" "B.Cu") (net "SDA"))
 (via (at 3.5966 8.5896) (size 0.6) (drill 0.3) (layers "F.Cu" "B.Cu") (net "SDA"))
 (segment (start -1.3923 7.9331) (end -0.7358 8.5896) (width 0.2) (layer "B.Cu") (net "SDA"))
 (segment (start 1.1351 -2.2384) (end -0.1009 -2.2384) (width 0.2) (layer "B.Cu") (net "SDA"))
 (segment (start -0.1009 -2.2384) (end -0.1375 -2.275) (width 0.2) (layer "B.Cu") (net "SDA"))
 (segment (start -1.0094 7) (end -1.3923 7.3829) (width 0.2) (layer "B.Cu") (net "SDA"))
 (segment (start -0.7358 8.5896) (end 3.5966 8.5896) (width 0.2) (layer "B.Cu") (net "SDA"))
 (segment (start 1.1351 0.3837) (end 0.5438 0.975) (width 0.2) (layer "B.Cu") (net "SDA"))
 (segment (start 0.5438 0.975) (end -0.1375 0.975) (width 0.2) (layer "B.Cu") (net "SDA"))
 (segment (start 1.1351 -2.2384) (end 1.1351 0.3837) (width 0.2) (layer "B.Cu") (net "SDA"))
 (segment (start -1.3923 7.3829) (end -1.3923 7.9331) (width 0.2) (layer "B.Cu") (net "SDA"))
 (segment (start -0.8875 7) (end -1.0094 7) (width 0.2) (layer "B.Cu") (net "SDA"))
 (segment (start 4.396 -3.3226) (end 8.825 -7.7516) (width 0.2) (layer "F.Cu") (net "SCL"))
 (segment (start 8.825 -7.7516) (end 8.825 -8) (width 0.2) (layer "F.Cu") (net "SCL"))
 (segment (start 1.0899 -3.3226) (end 4.396 -3.3226) (width 0.2) (layer "F.Cu") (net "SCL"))
 (via (at 1.0899 -3.3226) (size 0.6) (drill 0.3) (layers "F.Cu" "B.Cu") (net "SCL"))
 (segment (start 1.8166 8.1699) (end -0.5718 8.1699) (width 0.2) (layer "B.Cu") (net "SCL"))
 (segment (start 1.7531 -2.6594) (end 1.0899 -3.3226) (width 0.2) (layer "B.Cu") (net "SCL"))
 (segment (start -0.5718 8.1699) (end -0.8875 7.8542) (width 0.2) (layer "B.Cu") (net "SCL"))
 (segment (start -0.1375 1.625) (end 0.5673 1.625) (width 0.2) (layer "B.Cu") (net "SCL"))
 (segment (start 0.5673 1.625) (end 1.7531 0.4392) (width 0.2) (layer "B.Cu") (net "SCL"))
 (segment (start 1.0899 -3.3226) (end 0.2601 -3.3226) (width 0.2) (layer "B.Cu") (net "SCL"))
 (segment (start 0.5673 1.625) (end 2.214 3.2717) (width 0.2) (layer "B.Cu") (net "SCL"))
 (segment (start 1.7531 0.4392) (end 1.7531 -2.6594) (width 0.2) (layer "B.Cu") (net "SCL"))
 (segment (start 0.2601 -3.3226) (end -0.1375 -2.925) (width 0.2) (layer "B.Cu") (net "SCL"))
 (segment (start -0.8875 7.8542) (end -0.8875 7.65) (width 0.2) (layer "B.Cu") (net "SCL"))
 (segment (start 2.214 3.2717) (end 2.214 7.7725) (width 0.2) (layer "B.Cu") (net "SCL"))
 (segment (start 2.214 7.7725) (end 1.8166 8.1699) (width 0.2) (layer "B.Cu") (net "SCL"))
 (segment (start -6.825 -1.9252) (end -7.1252 -1.625) (width 0.2) (layer "F.Cu") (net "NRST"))
 (segment (start -6.825 -5) (end -6.825 -1.9252) (width 0.2) (layer "F.Cu") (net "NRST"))
 (via (at -7.1252 -1.625) (size 0.6) (drill 0.3) (layers "F.Cu" "B.Cu") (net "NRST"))
 (segment (start -5.8625 -1.625) (end -7.1252 -1.625) (width 0.2) (layer "B.Cu") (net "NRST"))
 (segment (start 13.1 -3.85) (end 9.9756 -3.85) (width 0.2) (layer "F.Cu") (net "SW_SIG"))
 (segment (start 9.9756 -3.85) (end 6.9 -3.85) (width 0.2) (layer "F.Cu") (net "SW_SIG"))
 (via (at 9.9756 -3.85) (size 0.6) (drill 0.3) (layers "F.Cu" "B.Cu") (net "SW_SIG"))
 (segment (start -1.2055 -3.195) (end -0.4762 -3.9243) (width 0.2) (layer "B.Cu") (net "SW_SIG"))
 (segment (start -0.1375 -1.625) (end -0.6666 -1.625) (width 0.2) (layer "B.Cu") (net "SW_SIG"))
 (segment (start 2.1533 -3.3112) (end 9.4368 -3.3112) (width 0.2) (layer "B.Cu") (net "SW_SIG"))
 (segment (start -2.0393 -1.625) (end -3.3393 -0.325) (width 0.2) (layer "B.Cu") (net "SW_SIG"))
 (segment (start -0.6666 -1.625) (end -2.0393 -1.625) (width 0.2) (layer "B.Cu") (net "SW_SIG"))
 (segment (start 9.4368 -3.3112) (end 9.9756 -3.85) (width 0.2) (layer "B.Cu") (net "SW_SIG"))
 (segment (start -0.4762 -3.9243) (end 1.5402 -3.9243) (width 0.2) (layer "B.Cu") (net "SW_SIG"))
 (segment (start -0.8248 -1.625) (end -1.2055 -2.0057) (width 0.2) (layer "B.Cu") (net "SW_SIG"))
 (segment (start 1.5402 -3.9243) (end 2.1533 -3.3112) (width 0.2) (layer "B.Cu") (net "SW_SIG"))
 (segment (start -3.3393 -0.325) (end -5.8625 -0.325) (width 0.2) (layer "B.Cu") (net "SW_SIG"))
 (segment (start -0.6666 -1.625) (end -0.8248 -1.625) (width 0.2) (layer "B.Cu") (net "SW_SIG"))
 (segment (start -1.2055 -2.0057) (end -1.2055 -3.195) (width 0.2) (layer "B.Cu") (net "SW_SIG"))
 (segment (start -0.6974 1.4714) (end -1.0575 1.8315) (width 0.2) (layer "F.Cu") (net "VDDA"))
 (segment (start -2.0114 -2.7756) (end -0.6974 -1.4616) (width 0.2) (layer "F.Cu") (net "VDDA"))
 (segment (start -1.0575 1.8315) (end -1.3809 1.8315) (width 0.2) (layer "F.Cu") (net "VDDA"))
 (segment (start -0.6974 -1.4616) (end -0.6974 1.4714) (width 0.2) (layer "F.Cu") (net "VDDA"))
 (segment (start -4.2788 -2.7756) (end -2.0114 -2.7756) (width 0.2) (layer "F.Cu") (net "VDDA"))
 (via (at -1.3809 1.8315) (size 0.6) (drill 0.3) (layers "F.Cu" "B.Cu") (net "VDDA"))
 (via (at -4.2788 -2.7756) (size 0.6) (drill 0.3) (layers "F.Cu" "B.Cu") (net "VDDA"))
 (segment (start -0.881 -0.325) (end -1.3809 0.1749) (width 0.2) (layer "B.Cu") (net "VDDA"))
 (segment (start -0.0544 -7) (end 2.725 -7) (width 0.2) (layer "B.Cu") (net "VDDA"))
 (segment (start -1.3809 0.1749) (end -1.3809 1.8315) (width 0.2) (layer "B.Cu") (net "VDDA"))
 (segment (start -4.2788 -2.7756) (end -0.0544 -7) (width 0.2) (layer "B.Cu") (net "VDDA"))
 (segment (start -5.7131 -2.7756) (end -5.8625 -2.925) (width 0.2) (layer "B.Cu") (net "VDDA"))
 (segment (start -4.2788 -2.7756) (end -5.7131 -2.7756) (width 0.2) (layer "B.Cu") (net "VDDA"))
 (segment (start -0.1375 -0.325) (end -0.881 -0.325) (width 0.2) (layer "B.Cu") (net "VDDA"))
 (segment (start 0.8875 7) (end 0.8875 6.35) (width 0.2) (layer "B.Cu") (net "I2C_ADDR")))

